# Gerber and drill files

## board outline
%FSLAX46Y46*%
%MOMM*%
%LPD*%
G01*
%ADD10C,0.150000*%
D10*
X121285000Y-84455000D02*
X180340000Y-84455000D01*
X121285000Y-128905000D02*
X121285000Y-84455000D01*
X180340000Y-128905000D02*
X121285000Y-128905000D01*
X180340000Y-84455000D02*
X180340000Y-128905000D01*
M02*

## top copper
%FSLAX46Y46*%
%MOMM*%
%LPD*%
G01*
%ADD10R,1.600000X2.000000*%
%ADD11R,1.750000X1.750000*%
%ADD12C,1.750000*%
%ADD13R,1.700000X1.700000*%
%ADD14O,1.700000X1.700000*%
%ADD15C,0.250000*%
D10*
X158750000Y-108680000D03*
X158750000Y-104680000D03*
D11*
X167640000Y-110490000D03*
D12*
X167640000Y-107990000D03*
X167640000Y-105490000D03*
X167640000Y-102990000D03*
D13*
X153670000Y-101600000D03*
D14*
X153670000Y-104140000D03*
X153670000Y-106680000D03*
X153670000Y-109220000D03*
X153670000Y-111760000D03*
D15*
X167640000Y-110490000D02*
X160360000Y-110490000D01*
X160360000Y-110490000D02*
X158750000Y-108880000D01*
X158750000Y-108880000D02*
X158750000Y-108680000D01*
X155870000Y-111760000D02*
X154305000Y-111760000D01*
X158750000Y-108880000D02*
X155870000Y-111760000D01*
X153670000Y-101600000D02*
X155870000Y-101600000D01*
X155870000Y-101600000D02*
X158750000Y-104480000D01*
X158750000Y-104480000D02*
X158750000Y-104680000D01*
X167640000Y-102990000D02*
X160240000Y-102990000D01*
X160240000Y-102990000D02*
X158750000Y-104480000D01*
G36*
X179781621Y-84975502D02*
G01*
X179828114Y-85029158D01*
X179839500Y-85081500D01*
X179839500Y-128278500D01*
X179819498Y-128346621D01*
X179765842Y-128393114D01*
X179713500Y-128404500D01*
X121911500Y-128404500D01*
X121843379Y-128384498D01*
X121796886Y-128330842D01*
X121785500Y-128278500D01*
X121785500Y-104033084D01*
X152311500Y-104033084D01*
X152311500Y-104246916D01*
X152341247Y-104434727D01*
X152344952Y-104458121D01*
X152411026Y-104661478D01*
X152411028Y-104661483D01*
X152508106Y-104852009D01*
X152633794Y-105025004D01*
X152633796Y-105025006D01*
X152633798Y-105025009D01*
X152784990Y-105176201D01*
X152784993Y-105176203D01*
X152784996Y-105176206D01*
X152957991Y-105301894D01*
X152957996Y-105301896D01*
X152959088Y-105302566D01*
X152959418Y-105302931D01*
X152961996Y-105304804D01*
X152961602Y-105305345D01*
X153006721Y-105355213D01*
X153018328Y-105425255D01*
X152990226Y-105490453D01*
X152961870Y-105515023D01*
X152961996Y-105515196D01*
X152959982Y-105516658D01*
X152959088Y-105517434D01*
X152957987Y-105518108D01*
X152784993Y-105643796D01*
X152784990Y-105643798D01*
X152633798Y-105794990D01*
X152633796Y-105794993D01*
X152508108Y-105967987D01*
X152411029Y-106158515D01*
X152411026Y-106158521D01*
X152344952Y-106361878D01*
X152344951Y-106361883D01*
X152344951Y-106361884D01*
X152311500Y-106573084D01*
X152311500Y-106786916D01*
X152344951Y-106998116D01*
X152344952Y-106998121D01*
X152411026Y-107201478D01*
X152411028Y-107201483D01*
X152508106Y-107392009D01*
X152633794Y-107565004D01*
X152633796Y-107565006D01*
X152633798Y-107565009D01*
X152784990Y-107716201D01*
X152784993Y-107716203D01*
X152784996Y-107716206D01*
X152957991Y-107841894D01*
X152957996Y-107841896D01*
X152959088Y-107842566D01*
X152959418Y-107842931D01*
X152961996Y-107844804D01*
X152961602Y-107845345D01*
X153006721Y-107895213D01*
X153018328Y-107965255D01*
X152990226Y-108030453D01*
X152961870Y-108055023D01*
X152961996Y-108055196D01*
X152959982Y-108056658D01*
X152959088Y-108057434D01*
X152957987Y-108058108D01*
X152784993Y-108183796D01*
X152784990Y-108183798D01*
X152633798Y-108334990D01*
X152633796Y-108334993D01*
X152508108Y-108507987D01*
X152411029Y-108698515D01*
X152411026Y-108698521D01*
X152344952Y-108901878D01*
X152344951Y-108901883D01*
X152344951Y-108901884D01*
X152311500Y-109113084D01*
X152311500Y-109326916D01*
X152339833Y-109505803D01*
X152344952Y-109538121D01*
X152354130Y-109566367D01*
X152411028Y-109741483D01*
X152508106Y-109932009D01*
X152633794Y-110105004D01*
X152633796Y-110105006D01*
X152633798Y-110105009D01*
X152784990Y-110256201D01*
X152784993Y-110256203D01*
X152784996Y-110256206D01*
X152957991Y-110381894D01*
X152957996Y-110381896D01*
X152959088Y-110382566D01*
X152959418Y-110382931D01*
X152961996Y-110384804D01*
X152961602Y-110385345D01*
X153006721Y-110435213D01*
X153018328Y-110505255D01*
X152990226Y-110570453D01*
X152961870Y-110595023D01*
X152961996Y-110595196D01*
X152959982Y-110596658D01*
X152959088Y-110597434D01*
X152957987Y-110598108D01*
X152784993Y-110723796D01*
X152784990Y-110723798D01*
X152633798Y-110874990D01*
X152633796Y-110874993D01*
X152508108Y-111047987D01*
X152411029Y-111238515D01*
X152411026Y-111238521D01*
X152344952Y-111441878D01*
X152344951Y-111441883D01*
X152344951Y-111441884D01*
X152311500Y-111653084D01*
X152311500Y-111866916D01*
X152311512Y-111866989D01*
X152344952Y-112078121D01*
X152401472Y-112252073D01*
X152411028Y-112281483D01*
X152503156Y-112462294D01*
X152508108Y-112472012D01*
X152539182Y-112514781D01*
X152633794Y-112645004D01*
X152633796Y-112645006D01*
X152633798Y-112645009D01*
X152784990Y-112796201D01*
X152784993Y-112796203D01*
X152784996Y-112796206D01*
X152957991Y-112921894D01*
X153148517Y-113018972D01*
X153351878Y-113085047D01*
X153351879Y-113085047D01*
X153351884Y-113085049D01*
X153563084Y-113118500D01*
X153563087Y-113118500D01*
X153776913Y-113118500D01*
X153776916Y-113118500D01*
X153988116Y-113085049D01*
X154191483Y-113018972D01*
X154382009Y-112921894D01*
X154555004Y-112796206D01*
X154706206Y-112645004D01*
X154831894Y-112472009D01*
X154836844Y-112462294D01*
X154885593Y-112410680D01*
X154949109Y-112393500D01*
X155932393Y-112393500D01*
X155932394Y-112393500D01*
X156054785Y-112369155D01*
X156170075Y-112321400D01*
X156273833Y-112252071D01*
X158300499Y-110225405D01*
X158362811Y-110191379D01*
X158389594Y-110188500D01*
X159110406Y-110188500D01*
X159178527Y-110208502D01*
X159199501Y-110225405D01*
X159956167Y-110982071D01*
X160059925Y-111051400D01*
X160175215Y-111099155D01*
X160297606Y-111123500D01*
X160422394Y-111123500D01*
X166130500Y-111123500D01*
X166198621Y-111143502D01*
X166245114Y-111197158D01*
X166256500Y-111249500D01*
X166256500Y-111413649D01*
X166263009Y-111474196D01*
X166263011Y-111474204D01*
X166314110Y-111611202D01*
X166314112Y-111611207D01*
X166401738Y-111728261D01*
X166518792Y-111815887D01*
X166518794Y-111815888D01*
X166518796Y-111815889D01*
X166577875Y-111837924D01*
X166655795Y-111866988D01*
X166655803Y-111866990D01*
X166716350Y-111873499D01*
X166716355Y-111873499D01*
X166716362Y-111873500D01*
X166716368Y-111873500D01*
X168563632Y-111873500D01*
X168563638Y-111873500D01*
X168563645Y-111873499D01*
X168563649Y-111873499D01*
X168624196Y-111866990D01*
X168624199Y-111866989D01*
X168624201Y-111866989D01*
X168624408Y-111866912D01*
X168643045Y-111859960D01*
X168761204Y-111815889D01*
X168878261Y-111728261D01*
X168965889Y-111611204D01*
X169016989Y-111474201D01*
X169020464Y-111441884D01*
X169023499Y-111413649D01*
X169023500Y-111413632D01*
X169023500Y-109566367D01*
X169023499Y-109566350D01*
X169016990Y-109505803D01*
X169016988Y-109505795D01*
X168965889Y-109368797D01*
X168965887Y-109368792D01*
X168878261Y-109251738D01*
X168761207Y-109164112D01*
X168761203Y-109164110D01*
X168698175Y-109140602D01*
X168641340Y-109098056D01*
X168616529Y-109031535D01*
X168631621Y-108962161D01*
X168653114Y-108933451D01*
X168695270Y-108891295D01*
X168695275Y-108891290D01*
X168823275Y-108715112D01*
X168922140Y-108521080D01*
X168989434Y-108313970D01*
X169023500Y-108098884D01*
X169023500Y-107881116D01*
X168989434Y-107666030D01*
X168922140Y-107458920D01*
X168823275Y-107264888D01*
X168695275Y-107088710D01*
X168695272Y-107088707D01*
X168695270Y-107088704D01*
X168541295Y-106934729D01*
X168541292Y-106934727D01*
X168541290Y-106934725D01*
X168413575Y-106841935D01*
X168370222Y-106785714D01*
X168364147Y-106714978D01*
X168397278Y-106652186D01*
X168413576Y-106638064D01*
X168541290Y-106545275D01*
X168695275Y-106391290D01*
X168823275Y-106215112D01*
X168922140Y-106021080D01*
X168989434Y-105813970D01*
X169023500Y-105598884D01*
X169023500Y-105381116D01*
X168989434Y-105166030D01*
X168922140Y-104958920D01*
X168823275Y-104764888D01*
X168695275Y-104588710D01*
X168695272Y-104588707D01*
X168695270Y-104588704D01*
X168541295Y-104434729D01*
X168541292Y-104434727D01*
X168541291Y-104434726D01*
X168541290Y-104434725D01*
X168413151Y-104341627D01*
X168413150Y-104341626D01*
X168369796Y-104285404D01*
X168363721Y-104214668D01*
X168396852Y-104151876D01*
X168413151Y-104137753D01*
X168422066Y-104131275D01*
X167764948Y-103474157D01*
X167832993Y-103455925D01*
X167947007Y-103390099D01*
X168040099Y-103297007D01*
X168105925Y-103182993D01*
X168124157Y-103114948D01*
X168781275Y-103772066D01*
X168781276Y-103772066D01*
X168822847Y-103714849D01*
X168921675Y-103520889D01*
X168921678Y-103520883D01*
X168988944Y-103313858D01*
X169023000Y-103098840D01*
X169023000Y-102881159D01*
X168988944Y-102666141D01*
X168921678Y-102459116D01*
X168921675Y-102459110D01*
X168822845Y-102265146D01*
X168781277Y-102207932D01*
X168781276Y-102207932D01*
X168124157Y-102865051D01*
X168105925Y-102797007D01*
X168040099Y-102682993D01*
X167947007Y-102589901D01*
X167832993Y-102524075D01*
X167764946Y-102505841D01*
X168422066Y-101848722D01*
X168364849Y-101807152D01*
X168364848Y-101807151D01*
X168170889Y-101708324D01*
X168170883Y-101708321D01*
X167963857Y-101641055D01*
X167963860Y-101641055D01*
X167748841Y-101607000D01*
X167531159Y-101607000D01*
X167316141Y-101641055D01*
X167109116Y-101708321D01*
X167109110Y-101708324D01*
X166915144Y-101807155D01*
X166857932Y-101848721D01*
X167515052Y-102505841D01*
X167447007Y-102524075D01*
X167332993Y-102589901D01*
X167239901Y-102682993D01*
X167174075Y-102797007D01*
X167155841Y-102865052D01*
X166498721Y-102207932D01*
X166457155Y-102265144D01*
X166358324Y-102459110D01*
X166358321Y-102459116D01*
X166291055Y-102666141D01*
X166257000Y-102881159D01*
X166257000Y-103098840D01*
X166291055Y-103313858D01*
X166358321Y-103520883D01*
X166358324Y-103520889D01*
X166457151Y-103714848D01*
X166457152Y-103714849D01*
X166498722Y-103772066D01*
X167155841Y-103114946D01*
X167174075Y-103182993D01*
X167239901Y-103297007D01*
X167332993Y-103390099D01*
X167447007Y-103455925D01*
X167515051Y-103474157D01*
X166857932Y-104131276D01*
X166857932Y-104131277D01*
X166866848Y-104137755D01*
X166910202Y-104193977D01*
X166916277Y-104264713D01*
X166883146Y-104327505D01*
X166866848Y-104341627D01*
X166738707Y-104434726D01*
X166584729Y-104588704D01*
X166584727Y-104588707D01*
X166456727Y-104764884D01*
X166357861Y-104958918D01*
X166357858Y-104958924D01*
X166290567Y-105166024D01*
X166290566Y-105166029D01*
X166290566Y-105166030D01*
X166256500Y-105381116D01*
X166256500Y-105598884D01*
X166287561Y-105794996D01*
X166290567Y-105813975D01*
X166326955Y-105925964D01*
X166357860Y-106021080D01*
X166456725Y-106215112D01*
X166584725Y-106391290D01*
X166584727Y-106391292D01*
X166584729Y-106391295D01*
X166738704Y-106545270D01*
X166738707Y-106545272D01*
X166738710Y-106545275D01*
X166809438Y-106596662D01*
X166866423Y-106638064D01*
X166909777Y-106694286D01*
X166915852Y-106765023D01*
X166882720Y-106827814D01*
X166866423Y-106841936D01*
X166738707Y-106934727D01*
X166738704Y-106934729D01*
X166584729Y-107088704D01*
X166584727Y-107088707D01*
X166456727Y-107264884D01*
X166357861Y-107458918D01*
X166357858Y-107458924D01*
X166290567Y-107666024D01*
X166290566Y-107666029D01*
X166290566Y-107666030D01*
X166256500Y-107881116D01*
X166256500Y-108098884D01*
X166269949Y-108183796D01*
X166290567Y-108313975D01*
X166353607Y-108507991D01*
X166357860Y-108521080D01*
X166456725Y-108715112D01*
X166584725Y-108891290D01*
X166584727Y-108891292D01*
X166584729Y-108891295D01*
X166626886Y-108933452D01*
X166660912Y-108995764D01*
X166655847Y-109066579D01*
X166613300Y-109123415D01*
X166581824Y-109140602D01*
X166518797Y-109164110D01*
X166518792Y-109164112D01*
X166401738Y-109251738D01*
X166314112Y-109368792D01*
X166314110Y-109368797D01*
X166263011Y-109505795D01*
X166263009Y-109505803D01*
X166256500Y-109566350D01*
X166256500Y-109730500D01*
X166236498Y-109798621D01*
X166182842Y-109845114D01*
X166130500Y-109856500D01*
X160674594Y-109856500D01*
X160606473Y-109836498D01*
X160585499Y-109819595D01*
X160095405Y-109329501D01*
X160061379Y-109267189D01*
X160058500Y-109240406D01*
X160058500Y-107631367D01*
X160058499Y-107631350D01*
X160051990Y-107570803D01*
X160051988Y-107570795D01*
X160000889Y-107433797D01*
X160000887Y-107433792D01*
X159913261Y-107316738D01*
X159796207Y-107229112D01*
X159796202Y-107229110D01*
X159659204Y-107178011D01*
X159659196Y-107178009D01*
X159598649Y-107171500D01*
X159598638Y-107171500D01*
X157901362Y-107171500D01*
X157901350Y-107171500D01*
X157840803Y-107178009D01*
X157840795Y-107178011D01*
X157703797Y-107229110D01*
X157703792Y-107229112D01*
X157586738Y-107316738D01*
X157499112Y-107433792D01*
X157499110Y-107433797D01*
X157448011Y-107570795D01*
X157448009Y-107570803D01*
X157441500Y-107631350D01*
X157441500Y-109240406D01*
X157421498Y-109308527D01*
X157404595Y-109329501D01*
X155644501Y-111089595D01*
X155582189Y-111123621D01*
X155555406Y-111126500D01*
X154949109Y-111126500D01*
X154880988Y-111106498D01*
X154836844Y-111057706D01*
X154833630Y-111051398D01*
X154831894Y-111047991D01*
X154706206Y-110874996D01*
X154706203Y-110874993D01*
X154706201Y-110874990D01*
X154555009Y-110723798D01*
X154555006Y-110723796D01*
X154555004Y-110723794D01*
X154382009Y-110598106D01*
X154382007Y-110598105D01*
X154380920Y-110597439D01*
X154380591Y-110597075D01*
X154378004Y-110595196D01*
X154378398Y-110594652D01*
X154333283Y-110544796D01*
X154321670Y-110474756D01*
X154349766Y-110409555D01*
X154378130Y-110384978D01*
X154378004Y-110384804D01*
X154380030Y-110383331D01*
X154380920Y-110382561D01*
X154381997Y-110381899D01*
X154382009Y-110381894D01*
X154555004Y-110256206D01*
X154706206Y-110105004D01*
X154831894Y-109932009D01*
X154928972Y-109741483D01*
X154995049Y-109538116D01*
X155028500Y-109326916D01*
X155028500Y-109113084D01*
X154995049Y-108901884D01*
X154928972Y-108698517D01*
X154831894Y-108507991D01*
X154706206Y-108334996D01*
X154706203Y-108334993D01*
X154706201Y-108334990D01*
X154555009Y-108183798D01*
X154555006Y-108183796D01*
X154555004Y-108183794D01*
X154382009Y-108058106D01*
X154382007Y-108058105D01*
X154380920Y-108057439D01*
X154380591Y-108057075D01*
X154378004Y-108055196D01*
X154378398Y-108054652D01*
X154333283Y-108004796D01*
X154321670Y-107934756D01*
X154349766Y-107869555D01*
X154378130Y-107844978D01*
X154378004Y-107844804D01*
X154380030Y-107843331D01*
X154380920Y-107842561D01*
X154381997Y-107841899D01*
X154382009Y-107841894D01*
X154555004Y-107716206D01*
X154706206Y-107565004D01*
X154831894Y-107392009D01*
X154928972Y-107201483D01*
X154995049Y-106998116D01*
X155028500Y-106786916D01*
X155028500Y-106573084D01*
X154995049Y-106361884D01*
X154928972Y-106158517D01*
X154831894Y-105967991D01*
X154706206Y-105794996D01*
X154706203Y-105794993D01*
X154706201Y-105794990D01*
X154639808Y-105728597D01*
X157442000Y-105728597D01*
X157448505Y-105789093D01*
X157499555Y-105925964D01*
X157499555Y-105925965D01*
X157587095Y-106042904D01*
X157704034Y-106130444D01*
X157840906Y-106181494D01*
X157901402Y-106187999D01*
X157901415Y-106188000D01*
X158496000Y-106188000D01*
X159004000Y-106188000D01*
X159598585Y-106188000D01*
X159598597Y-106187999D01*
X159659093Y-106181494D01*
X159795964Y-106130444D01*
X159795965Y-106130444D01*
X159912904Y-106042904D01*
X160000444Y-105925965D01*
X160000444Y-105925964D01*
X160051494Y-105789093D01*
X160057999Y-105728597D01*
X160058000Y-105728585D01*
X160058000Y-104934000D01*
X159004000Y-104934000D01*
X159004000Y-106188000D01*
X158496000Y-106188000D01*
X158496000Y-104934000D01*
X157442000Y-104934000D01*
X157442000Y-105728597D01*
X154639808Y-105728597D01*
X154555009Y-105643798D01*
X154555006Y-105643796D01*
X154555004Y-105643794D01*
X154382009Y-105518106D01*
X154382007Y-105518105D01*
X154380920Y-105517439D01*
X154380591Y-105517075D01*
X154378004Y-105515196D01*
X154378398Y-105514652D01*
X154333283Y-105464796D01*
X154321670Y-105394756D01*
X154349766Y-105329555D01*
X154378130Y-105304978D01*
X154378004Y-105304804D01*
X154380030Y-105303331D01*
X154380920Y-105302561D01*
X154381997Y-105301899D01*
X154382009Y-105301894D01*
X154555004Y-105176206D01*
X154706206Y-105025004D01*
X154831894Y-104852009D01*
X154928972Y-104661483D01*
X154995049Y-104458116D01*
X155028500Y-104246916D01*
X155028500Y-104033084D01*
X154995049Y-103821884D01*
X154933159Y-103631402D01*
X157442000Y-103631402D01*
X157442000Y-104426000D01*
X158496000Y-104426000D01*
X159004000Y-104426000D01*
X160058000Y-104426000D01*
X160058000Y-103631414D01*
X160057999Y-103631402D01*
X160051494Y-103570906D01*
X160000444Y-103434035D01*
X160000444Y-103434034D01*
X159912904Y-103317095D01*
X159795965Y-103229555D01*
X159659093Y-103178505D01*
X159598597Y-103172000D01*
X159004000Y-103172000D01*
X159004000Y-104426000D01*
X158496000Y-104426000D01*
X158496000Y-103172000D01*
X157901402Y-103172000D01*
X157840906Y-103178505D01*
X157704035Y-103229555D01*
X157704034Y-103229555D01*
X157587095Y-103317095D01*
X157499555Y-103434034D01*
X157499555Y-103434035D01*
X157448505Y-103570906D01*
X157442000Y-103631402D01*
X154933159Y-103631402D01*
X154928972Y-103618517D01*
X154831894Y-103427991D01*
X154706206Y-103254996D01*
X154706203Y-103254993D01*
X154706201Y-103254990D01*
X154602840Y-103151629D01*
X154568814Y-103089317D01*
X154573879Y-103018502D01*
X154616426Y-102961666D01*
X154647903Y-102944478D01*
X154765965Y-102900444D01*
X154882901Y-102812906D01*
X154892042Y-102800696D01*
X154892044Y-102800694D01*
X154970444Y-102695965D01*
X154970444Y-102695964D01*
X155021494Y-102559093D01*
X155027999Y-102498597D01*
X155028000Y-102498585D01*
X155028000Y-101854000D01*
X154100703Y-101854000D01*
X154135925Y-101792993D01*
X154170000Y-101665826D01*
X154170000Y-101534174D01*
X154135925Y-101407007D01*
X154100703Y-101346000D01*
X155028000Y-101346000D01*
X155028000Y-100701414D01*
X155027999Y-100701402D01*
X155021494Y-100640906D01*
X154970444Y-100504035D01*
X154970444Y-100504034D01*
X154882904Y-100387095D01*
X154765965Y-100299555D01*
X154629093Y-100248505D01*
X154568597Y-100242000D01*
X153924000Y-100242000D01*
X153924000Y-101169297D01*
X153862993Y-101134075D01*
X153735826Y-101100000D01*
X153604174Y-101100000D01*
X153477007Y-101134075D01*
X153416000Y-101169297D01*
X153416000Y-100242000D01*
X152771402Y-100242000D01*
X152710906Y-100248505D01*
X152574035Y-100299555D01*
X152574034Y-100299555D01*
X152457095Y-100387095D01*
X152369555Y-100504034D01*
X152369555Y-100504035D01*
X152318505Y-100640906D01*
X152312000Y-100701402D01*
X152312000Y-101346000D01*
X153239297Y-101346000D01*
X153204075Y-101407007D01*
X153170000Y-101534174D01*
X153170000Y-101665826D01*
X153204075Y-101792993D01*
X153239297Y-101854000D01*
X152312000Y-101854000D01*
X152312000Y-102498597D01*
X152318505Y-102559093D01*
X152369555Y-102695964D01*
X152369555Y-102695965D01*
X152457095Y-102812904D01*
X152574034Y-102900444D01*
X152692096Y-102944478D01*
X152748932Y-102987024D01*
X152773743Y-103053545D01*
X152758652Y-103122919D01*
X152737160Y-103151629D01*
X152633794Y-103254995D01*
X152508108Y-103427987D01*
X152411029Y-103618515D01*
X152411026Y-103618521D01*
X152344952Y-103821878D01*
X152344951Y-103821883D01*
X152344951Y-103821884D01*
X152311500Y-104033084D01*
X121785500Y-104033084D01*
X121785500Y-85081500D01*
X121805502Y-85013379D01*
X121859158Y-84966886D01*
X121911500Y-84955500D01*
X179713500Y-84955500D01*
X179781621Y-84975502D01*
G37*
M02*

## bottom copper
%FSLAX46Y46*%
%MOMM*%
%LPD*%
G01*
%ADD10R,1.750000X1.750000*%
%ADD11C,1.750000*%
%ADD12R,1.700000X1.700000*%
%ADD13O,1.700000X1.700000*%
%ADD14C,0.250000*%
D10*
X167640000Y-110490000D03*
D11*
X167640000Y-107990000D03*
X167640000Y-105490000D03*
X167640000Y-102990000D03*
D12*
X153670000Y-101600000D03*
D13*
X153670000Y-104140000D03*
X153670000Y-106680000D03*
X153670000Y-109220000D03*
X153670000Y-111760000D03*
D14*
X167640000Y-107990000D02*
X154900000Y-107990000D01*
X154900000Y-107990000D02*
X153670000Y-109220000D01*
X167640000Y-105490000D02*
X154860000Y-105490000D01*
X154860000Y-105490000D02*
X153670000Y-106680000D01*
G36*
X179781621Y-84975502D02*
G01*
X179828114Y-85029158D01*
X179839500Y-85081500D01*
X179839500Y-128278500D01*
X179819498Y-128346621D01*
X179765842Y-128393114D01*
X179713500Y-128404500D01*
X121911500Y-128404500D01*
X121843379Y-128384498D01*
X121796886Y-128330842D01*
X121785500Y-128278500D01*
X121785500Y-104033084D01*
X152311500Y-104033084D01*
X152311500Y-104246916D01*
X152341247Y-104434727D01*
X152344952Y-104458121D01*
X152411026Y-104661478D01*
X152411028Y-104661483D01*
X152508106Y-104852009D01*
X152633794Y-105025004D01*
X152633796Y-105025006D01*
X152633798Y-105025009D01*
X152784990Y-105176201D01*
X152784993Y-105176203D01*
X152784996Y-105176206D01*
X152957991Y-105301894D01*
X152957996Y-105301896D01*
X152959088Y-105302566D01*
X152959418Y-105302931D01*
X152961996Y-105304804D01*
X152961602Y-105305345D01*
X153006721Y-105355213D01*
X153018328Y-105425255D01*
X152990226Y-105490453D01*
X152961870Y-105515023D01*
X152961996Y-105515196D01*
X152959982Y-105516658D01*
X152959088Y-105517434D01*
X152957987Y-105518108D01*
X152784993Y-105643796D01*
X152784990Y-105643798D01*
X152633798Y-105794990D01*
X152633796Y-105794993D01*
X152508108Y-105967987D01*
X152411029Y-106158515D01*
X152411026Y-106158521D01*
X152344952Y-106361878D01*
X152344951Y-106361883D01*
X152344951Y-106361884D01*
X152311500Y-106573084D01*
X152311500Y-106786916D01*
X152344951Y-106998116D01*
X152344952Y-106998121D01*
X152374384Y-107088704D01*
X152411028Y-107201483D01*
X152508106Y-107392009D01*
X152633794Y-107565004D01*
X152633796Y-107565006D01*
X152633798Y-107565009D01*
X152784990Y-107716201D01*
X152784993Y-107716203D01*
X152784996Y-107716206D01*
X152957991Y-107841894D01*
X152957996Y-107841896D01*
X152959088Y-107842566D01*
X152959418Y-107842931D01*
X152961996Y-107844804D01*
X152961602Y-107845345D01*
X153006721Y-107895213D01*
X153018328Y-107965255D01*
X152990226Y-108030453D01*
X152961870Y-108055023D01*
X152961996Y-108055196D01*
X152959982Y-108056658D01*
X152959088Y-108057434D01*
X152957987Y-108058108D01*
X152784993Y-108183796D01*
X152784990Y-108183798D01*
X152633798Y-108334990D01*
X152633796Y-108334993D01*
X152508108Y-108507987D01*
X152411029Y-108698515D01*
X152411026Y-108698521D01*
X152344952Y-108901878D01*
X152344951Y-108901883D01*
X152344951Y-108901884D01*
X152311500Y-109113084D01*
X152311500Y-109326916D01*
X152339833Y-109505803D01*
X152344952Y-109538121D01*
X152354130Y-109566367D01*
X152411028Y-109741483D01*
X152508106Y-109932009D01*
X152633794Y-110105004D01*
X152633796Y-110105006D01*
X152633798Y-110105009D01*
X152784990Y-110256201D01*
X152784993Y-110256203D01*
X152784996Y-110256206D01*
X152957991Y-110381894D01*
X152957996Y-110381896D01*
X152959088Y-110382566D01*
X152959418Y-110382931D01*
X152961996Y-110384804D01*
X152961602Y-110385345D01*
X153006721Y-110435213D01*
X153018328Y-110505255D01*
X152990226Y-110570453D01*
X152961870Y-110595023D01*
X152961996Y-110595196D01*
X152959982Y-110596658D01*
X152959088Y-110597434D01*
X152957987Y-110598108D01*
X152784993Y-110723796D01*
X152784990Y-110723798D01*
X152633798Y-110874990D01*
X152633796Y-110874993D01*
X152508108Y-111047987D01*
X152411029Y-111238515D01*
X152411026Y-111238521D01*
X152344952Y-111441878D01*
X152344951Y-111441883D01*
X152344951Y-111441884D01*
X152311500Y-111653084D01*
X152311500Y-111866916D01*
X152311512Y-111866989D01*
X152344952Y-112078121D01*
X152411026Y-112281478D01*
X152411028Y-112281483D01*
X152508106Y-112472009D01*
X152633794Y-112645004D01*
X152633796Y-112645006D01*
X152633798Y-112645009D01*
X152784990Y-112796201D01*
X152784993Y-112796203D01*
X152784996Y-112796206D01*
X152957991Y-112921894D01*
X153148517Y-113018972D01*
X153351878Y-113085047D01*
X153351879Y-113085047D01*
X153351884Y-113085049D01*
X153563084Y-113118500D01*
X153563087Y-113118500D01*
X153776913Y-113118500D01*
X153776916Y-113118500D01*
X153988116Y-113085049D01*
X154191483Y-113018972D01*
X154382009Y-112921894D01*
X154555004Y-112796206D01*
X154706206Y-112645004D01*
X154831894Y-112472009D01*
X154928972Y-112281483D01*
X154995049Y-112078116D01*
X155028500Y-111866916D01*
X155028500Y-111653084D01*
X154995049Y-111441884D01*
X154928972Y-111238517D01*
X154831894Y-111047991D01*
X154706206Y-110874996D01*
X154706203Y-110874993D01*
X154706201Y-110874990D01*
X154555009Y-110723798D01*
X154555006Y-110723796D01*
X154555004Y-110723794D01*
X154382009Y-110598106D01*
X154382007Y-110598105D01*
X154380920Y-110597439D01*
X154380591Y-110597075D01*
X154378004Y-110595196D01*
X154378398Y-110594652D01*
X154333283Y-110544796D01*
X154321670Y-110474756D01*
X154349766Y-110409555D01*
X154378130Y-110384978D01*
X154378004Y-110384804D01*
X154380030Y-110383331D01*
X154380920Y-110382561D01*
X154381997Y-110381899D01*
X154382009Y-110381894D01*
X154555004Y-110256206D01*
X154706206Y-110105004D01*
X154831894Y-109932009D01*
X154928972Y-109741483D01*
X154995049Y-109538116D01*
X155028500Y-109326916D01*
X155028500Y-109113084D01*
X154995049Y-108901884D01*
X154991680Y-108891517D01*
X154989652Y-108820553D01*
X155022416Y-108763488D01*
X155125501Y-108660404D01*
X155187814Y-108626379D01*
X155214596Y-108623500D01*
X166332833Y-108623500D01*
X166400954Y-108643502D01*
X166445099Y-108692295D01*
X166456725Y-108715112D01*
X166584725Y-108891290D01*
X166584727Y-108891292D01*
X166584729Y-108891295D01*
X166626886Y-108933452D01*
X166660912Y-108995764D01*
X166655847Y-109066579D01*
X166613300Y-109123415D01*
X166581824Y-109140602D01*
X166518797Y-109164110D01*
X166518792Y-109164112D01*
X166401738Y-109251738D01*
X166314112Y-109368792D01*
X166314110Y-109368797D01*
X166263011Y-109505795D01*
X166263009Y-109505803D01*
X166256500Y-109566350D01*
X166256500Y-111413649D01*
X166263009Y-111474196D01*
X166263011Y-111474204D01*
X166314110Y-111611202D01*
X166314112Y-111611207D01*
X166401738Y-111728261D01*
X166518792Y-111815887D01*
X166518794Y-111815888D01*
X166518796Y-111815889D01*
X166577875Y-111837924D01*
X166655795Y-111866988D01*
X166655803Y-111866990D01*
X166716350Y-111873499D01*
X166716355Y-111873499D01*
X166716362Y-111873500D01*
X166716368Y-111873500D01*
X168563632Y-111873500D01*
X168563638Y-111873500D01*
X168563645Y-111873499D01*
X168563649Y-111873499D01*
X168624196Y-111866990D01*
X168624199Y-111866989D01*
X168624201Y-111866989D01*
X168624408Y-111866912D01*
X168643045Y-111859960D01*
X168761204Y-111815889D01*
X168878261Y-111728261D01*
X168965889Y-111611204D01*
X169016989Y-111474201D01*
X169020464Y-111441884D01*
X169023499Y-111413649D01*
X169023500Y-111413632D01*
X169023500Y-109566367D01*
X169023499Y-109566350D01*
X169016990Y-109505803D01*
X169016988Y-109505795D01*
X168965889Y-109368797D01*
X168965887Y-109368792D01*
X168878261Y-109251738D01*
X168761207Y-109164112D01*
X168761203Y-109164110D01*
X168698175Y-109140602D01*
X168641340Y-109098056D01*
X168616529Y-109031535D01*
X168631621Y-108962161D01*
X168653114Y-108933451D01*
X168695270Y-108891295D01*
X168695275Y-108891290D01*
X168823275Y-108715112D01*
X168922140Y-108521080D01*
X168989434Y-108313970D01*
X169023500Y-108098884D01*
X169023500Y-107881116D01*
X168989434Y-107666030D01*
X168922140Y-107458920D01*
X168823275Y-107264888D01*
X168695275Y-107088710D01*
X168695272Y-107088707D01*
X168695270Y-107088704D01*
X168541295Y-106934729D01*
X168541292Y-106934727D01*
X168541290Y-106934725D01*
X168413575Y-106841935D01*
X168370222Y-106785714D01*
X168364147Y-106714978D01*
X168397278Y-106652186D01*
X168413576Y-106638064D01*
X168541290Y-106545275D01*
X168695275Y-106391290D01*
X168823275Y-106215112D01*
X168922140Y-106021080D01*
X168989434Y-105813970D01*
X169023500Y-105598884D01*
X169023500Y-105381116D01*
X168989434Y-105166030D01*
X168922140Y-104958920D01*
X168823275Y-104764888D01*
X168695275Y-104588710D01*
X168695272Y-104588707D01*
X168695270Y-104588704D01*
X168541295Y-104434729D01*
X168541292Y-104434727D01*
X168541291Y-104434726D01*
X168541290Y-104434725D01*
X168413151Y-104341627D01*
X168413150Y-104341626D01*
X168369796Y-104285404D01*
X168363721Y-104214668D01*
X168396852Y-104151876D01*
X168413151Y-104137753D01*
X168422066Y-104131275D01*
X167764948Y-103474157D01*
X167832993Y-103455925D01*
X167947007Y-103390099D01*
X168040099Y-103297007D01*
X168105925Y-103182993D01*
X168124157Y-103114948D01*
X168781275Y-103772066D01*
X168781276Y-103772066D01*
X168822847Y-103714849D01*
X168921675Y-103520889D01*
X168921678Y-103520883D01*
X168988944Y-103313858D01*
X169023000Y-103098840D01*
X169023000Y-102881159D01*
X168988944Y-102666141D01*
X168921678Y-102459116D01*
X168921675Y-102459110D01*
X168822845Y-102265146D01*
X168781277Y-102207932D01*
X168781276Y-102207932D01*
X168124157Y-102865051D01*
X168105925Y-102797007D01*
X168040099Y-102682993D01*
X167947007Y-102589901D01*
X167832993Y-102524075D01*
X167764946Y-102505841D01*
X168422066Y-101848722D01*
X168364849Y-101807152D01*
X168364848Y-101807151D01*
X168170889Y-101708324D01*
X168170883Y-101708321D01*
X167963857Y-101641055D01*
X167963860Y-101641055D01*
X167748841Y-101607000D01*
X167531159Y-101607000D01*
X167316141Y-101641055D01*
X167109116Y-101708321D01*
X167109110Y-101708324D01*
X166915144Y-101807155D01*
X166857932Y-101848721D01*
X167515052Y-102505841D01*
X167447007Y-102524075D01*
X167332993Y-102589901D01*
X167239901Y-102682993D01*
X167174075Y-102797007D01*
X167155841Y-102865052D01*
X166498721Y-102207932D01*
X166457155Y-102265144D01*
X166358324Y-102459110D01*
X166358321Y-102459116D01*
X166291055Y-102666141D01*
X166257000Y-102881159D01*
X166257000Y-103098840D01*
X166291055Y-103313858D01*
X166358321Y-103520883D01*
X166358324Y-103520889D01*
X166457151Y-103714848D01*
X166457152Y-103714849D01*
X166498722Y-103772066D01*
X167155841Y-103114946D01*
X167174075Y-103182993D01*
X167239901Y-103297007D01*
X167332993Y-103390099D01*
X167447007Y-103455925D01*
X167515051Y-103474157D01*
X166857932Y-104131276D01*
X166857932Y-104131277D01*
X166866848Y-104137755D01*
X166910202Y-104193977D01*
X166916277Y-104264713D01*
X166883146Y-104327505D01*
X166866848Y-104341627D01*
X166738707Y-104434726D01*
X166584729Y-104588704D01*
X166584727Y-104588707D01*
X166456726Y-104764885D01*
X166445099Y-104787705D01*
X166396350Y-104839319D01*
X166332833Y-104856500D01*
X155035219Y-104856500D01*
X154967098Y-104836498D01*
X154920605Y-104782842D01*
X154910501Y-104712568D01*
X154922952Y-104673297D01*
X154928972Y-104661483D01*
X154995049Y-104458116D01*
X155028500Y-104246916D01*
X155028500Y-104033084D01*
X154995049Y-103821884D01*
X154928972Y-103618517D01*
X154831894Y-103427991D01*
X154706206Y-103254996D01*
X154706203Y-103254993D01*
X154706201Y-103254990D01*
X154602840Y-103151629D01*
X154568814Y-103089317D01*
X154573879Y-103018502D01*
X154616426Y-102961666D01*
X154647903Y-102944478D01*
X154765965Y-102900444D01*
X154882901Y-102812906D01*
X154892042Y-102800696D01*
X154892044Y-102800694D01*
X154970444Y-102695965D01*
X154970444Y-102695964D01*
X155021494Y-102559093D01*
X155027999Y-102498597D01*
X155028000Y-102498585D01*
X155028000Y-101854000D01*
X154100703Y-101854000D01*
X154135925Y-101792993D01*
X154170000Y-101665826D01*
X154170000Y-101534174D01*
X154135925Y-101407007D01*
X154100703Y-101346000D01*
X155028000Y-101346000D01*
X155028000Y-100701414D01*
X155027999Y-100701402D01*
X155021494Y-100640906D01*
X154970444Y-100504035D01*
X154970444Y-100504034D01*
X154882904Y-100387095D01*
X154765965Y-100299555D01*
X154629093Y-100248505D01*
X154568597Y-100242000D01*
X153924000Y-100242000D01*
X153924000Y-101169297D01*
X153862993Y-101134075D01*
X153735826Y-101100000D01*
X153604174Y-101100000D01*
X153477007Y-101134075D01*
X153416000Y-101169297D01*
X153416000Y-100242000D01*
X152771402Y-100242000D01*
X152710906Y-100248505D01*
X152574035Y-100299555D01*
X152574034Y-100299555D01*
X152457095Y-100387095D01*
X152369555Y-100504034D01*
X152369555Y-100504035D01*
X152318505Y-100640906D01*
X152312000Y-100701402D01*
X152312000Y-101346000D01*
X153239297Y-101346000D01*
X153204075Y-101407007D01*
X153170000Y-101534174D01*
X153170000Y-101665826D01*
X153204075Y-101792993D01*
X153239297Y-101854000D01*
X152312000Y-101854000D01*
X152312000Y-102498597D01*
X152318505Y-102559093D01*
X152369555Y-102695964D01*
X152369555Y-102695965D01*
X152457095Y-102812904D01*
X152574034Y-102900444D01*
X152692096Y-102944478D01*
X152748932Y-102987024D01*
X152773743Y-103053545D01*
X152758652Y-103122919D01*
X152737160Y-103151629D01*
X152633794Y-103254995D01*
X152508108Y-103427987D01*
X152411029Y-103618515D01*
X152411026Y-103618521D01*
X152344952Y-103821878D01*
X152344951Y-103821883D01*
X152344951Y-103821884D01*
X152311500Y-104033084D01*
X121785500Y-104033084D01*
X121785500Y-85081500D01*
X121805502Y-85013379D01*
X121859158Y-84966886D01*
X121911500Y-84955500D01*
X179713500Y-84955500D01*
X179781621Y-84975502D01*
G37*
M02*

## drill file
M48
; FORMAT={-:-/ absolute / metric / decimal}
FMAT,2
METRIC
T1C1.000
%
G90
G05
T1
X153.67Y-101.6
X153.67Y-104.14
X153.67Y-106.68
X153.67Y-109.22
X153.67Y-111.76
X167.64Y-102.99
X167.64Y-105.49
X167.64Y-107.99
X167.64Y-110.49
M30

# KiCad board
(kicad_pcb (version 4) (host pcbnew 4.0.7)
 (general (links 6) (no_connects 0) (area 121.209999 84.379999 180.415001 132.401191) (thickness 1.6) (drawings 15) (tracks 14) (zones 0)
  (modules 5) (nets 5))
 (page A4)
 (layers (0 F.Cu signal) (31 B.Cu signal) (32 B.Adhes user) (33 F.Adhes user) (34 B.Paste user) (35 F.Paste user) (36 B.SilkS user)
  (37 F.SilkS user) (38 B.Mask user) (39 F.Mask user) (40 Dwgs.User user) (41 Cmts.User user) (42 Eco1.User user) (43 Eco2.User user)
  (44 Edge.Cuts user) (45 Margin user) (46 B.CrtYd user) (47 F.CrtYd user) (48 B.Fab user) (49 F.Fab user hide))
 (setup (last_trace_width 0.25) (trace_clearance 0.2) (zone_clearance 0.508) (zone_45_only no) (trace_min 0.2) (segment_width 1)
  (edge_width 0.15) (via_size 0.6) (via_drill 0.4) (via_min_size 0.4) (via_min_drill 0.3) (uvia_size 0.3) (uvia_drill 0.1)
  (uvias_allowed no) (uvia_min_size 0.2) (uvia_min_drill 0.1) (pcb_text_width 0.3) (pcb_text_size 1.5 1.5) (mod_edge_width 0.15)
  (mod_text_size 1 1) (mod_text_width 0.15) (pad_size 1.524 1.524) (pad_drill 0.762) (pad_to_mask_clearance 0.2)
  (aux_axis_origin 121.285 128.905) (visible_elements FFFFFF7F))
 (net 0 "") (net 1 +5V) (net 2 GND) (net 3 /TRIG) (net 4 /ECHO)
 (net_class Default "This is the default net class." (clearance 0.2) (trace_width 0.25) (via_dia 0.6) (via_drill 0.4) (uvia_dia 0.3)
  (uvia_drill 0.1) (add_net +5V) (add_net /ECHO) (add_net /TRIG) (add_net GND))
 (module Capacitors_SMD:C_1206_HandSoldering (layer F.Cu) (at 158.75 106.68 90)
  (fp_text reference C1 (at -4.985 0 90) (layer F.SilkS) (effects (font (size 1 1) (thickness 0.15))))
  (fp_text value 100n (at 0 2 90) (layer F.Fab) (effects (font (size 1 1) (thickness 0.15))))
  (pad 1 smd rect (at -2 0 90) (size 2 1.6) (layers F.Cu F.Paste F.Mask) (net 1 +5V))
  (pad 2 smd rect (at 2 0 90) (size 2 1.6) (layers F.Cu F.Paste F.Mask) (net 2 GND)))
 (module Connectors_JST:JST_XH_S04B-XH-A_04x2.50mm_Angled (layer F.Cu) (at 167.64 110.49 90)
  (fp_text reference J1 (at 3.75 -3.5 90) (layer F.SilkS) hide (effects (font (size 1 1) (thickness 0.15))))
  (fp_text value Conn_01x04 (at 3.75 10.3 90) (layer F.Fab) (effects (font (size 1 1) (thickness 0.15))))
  (pad 1 thru_hole rect (at 0 0 90) (size 1.75 1.75) (drill 1) (layers *.Cu *.Mask F.SilkS) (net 1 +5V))
  (pad 2 thru_hole circle (at 2.5 0 90) (size 1.75 1.75) (drill 1) (layers *.Cu *.Mask F.SilkS) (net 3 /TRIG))
  (pad 3 thru_hole circle (at 5 0 90) (size 1.75 1.75) (drill 1) (layers *.Cu *.Mask F.SilkS) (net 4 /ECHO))
  (pad 4 thru_hole circle (at 7.5 0 90) (size 1.75 1.75) (drill 1) (layers *.Cu *.Mask F.SilkS) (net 2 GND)))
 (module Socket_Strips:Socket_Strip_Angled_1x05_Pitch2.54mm (layer F.Cu) (at 153.67 101.6)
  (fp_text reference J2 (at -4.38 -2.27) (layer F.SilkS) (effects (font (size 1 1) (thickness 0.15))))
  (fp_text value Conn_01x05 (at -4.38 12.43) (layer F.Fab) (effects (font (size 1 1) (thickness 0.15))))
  (pad 1 thru_hole rect (at 0 0) (size 1.7 1.7) (drill 1) (layers *.Cu *.Mask) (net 2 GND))
  (pad 2 thru_hole oval (at 0 2.54) (size 1.7 1.7) (drill 1) (layers *.Cu *.Mask))
  (pad 3 thru_hole oval (at 0 5.08) (size 1.7 1.7) (drill 1) (layers *.Cu *.Mask) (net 4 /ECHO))
  (pad 4 thru_hole oval (at 0 7.62) (size 1.7 1.7) (drill 1) (layers *.Cu *.Mask) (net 3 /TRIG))
  (pad 5 thru_hole oval (at 0 10.16) (size 1.7 1.7) (drill 1) (layers *.Cu *.Mask) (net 1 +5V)))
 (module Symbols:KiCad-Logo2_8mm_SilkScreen (layer B.Cu) (at 160.655 97.155 270)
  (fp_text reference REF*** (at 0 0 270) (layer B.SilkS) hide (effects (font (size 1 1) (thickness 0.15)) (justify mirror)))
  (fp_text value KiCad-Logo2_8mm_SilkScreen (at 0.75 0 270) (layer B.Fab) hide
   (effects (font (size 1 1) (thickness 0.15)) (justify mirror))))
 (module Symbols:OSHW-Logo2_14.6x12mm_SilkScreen (layer B.Cu) (at 160.02 117.475 270)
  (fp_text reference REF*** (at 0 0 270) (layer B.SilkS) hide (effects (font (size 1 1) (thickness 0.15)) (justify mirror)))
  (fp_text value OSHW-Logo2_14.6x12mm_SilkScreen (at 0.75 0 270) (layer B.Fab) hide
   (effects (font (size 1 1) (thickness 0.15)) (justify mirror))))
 (gr_line (start 121.285 84.455) (end 180.34 84.455) (layer Edge.Cuts) (width 0.15))
 (gr_line (start 121.285 128.905) (end 121.285 84.455) (layer Edge.Cuts) (width 0.15))
 (gr_line (start 180.34 128.905) (end 121.285 128.905) (layer Edge.Cuts) (width 0.15))
 (gr_line (start 180.34 84.455) (end 180.34 128.905) (layer Edge.Cuts) (width 0.15))
 (segment (start 167.64 110.49) (end 160.36 110.49) (width 0.25) (layer F.Cu) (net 1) (status 10))
 (segment (start 160.36 110.49) (end 158.75 108.88) (width 0.25) (layer F.Cu) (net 1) (status 20))
 (segment (start 158.75 108.88) (end 158.75 108.68) (width 0.25) (layer F.Cu) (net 1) (status 30))
 (segment (start 155.87 111.76) (end 154.305 111.76) (width 0.25) (layer F.Cu) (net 1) (status 20))
 (segment (start 158.75 108.88) (end 155.87 111.76) (width 0.25) (layer F.Cu) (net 1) (status 10))
 (segment (start 153.67 101.6) (end 155.87 101.6) (width 0.25) (layer F.Cu) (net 2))
 (segment (start 155.87 101.6) (end 158.75 104.48) (width 0.25) (layer F.Cu) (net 2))
 (segment (start 158.75 104.48) (end 158.75 104.68) (width 0.25) (layer F.Cu) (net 2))
 (segment (start 167.64 102.99) (end 160.24 102.99) (width 0.25) (layer F.Cu) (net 2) (status 10))
 (segment (start 160.24 102.99) (end 158.75 104.48) (width 0.25) (layer F.Cu) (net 2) (status 20))
 (segment (start 167.64 107.99) (end 154.9 107.99) (width 0.25) (layer B.Cu) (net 3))
 (segment (start 154.9 107.99) (end 153.67 109.22) (width 0.25) (layer B.Cu) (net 3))
 (segment (start 167.64 105.49) (end 154.86 105.49) (width 0.25) (layer B.Cu) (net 4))
 (segment (start 154.86 105.49) (end 153.67 106.68) (width 0.25) (layer B.Cu) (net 4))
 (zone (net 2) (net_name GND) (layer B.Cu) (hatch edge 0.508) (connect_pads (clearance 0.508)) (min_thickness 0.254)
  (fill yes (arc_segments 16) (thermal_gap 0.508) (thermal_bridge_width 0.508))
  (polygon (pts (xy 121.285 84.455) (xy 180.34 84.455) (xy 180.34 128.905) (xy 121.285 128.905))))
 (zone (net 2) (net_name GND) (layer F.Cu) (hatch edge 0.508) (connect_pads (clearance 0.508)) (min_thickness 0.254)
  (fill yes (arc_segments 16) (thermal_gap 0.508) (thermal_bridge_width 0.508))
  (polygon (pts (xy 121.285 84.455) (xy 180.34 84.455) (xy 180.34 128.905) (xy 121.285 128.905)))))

